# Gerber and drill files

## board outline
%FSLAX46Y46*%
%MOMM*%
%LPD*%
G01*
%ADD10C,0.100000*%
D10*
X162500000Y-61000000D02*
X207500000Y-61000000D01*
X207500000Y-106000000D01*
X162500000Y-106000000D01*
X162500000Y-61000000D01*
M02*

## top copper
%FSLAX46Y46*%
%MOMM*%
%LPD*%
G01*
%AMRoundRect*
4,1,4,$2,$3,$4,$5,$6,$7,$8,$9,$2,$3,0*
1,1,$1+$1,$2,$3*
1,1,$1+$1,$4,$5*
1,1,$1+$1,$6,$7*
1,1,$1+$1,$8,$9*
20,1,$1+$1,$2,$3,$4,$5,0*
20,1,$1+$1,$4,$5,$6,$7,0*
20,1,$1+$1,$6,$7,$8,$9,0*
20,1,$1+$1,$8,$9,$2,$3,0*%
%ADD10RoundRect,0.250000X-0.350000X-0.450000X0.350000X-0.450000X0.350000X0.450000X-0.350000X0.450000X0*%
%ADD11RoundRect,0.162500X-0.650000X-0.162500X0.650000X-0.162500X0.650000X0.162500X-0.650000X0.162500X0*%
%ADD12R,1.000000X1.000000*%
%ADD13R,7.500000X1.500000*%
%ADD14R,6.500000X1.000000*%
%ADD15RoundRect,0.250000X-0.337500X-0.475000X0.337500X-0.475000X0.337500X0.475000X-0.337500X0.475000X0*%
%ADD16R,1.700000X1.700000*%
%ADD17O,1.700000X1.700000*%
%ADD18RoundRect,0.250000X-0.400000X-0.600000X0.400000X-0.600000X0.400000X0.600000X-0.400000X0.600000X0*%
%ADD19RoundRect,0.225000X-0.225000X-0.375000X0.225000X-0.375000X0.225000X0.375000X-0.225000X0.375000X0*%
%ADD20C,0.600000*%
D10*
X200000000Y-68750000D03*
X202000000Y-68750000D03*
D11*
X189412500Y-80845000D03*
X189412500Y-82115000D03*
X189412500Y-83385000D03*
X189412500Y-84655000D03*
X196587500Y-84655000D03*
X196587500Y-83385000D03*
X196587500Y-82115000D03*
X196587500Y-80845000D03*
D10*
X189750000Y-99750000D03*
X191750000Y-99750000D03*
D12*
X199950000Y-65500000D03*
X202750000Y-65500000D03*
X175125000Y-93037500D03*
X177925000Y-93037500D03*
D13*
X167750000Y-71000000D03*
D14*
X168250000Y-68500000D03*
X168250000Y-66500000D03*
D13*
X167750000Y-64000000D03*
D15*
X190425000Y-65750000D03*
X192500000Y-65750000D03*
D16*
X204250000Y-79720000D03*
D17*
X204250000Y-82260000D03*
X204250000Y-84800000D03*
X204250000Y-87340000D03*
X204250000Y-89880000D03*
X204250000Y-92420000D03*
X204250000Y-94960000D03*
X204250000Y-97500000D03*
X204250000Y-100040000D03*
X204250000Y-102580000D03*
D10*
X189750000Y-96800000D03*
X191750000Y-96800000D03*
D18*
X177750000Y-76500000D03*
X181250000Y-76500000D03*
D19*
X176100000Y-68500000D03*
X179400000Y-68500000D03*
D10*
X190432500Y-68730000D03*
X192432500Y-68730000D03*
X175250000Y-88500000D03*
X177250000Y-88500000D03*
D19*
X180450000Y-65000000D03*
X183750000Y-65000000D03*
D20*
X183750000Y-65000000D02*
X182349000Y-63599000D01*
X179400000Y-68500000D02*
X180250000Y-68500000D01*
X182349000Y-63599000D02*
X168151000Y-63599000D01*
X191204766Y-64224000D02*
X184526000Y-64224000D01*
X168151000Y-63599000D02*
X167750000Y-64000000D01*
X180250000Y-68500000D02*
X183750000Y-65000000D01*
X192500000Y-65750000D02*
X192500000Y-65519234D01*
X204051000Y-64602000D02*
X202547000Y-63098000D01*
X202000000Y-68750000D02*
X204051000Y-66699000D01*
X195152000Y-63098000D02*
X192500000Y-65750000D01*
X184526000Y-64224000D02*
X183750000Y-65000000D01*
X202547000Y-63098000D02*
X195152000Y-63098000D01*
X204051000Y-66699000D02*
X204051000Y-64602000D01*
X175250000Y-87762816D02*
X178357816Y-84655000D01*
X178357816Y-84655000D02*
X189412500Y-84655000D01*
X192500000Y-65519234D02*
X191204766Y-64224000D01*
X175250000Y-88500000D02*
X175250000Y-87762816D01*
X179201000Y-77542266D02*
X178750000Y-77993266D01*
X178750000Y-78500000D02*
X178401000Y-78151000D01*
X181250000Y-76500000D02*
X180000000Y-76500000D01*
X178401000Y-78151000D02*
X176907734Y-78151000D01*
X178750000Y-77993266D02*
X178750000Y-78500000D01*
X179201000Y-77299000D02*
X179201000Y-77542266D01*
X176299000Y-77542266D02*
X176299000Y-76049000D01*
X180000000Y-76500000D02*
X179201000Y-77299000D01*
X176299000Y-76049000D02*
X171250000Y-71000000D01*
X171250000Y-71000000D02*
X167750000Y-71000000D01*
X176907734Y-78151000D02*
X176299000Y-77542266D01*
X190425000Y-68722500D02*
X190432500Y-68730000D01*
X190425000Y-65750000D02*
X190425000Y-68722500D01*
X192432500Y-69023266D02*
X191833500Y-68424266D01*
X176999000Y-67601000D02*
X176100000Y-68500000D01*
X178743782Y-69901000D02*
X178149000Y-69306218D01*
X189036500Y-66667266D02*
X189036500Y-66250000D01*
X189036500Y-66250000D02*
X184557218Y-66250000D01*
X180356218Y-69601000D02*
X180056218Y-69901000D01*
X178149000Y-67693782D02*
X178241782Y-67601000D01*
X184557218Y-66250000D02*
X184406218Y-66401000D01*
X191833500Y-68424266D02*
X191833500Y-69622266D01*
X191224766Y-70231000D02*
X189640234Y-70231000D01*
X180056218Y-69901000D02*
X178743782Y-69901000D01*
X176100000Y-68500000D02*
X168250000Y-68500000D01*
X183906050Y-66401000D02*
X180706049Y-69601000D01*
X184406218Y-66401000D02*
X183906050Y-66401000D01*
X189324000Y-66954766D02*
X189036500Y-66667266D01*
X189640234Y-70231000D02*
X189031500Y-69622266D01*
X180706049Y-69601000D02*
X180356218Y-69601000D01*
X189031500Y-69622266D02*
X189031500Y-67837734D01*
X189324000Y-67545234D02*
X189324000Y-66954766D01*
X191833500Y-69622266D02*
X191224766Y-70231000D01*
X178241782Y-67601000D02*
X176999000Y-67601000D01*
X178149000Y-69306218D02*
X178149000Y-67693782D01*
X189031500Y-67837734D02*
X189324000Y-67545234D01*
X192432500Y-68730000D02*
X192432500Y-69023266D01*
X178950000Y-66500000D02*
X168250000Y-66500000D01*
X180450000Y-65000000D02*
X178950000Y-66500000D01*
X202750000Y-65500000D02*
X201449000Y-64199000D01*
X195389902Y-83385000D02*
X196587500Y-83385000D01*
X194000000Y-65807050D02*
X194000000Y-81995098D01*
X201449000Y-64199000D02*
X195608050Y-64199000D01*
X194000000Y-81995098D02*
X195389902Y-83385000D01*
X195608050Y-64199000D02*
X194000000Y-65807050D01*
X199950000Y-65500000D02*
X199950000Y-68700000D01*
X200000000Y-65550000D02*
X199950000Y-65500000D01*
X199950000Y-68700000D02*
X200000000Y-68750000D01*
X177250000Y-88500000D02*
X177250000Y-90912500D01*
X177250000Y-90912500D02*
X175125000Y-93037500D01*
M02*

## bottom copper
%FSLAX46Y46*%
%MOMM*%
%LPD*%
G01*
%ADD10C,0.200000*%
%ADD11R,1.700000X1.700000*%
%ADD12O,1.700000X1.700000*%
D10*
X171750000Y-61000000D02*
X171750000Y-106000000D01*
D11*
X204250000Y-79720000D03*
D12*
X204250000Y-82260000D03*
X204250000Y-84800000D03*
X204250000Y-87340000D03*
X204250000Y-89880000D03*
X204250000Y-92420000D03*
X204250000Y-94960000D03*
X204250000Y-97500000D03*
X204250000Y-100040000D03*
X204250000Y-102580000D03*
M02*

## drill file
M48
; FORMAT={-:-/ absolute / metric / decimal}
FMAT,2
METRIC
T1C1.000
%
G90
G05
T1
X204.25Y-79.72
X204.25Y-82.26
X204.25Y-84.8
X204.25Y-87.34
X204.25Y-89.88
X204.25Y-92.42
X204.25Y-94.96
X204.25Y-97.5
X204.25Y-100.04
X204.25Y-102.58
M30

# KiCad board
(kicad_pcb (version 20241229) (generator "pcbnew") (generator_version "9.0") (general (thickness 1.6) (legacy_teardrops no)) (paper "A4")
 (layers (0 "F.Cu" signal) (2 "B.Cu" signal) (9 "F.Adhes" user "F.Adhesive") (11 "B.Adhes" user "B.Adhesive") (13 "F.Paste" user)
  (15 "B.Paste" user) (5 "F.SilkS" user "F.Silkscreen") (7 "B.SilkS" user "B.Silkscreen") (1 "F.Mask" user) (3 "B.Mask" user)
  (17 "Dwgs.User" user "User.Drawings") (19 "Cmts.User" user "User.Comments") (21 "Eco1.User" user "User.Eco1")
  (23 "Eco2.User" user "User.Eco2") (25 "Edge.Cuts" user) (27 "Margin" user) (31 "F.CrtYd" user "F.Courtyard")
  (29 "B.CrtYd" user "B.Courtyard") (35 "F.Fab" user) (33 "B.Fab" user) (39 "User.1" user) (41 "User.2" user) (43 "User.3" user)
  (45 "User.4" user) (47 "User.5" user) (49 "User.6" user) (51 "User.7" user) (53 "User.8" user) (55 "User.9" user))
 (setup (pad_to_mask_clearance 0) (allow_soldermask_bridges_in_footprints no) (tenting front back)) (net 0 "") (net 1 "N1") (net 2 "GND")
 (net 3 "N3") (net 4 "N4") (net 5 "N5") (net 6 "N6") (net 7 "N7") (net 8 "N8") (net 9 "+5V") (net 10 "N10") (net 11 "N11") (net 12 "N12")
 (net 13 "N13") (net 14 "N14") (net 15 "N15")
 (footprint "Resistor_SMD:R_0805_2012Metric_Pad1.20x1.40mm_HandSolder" (layer "F.Cu") (at 201 68.75)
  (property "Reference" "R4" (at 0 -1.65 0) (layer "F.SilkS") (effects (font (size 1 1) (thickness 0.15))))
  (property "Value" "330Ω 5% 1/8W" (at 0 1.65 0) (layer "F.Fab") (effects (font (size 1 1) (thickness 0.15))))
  (pad "1" smd roundrect (at -1 0) (size 1.2 1.4) (layers "F.Cu" "F.Mask" "F.Paste") (roundrect_rratio 0.208333) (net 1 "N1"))
  (pad "2" smd roundrect (at 1 0) (size 1.2 1.4) (layers "F.Cu" "F.Mask" "F.Paste") (roundrect_rratio 0.208333) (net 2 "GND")))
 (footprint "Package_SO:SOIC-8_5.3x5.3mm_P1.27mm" (layer "F.Cu") (at 193 82.75)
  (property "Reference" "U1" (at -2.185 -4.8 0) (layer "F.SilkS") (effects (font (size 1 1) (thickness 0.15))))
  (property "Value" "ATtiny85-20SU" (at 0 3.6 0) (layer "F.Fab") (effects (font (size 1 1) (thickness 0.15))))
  (pad "1" smd roundrect (at -3.5875 -1.905) (size 1.625 0.65) (layers "F.Cu" "F.Mask" "F.Paste") (roundrect_rratio 0.25) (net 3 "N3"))
  (pad "2" smd roundrect (at -3.5875 -0.635) (size 1.625 0.65) (layers "F.Cu" "F.Mask" "F.Paste") (roundrect_rratio 0.25) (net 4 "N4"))
  (pad "3" smd roundrect (at -3.5875 0.635) (size 1.625 0.65) (layers "F.Cu" "F.Mask" "F.Paste") (roundrect_rratio 0.25) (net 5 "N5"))
  (pad "4" smd roundrect (at -3.5875 1.905) (size 1.625 0.65) (layers "F.Cu" "F.Mask" "F.Paste") (roundrect_rratio 0.25) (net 2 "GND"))
  (pad "5" smd roundrect (at 3.5875 1.905) (size 1.625 0.65) (layers "F.Cu" "F.Mask" "F.Paste") (roundrect_rratio 0.25) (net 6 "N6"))
  (pad "6" smd roundrect (at 3.5875 0.635) (size 1.625 0.65) (layers "F.Cu" "F.Mask" "F.Paste") (roundrect_rratio 0.25) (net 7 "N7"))
  (pad "7" smd roundrect (at 3.5875 -0.635) (size 1.625 0.65) (layers "F.Cu" "F.Mask" "F.Paste") (roundrect_rratio 0.25) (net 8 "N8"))
  (pad "8" smd roundrect (at 3.5875 -1.905) (size 1.625 0.65) (layers "F.Cu" "F.Mask" "F.Paste") (roundrect_rratio 0.25) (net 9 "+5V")))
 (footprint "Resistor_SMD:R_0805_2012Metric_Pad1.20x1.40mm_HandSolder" (layer "F.Cu") (at 190.75 99.75)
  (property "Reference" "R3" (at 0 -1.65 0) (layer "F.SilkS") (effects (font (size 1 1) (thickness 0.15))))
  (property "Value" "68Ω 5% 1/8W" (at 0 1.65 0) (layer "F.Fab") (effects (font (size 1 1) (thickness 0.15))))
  (pad "1" smd roundrect (at -1 0) (size 1.2 1.4) (layers "F.Cu" "F.Mask" "F.Paste") (roundrect_rratio 0.208333) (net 5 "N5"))
  (pad "2" smd roundrect (at 1 0) (size 1.2 1.4) (layers "F.Cu" "F.Mask" "F.Paste") (roundrect_rratio 0.208333) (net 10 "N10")))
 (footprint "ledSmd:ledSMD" (layer "F.Cu") (at 201.75 65.5)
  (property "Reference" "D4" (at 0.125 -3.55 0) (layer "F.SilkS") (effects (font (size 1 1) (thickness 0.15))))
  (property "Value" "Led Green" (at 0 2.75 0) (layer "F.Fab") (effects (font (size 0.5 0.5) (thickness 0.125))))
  (pad "1" smd rect (at -1.8 0) (size 1 1) (layers "F.Cu" "F.Mask" "F.Paste") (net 1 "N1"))
  (pad "2" smd rect (at 1 0) (size 1 1) (layers "F.Cu" "F.Mask" "F.Paste") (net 7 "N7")))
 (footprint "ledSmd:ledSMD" (layer "F.Cu") (at 176.925 93.0375)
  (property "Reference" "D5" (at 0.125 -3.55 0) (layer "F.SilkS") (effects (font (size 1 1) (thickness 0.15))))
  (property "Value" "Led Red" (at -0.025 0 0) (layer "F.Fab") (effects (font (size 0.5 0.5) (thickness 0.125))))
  (pad "1" smd rect (at -1.8 0) (size 1 1) (layers "F.Cu" "F.Mask" "F.Paste") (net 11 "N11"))
  (pad "2" smd rect (at 1 0) (size 1 1) (layers "F.Cu" "F.Mask" "F.Paste") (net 9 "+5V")))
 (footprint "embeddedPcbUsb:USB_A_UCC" (layer "F.Cu") (at 167.95 67.5)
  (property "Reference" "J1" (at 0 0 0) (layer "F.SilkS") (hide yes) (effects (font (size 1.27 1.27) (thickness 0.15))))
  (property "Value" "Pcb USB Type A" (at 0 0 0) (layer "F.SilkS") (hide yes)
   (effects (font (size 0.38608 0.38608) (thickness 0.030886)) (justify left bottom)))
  (pad "1" smd rect (at -0.2 3.5) (size 7.5 1.5) (layers "F.Cu" "F.Mask" "F.Paste") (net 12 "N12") (solder_mask_margin 0.1016))
  (pad "2" smd rect (at 0.3 1) (size 6.5 1) (layers "F.Cu" "F.Mask" "F.Paste") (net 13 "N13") (solder_mask_margin 0.1016))
  (pad "3" smd rect (at 0.3 -1) (size 6.5 1) (layers "F.Cu" "F.Mask" "F.Paste") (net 10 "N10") (solder_mask_margin 0.1016))
  (pad "4" smd rect (at -0.2 -3.5) (size 7.5 1.5) (layers "F.Cu" "F.Mask" "F.Paste") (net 2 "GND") (solder_mask_margin 0.1016)))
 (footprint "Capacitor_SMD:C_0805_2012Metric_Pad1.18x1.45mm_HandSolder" (layer "F.Cu") (at 191.4625 65.75)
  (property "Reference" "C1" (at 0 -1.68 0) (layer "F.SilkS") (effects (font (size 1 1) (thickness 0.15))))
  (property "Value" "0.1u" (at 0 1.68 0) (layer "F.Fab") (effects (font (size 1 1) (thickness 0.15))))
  (pad "1" smd roundrect (at -1.0375 0) (size 1.175 1.45) (layers "F.Cu" "F.Mask" "F.Paste") (roundrect_rratio 0.212766) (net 9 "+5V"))
  (pad "2" smd roundrect (at 1.0375 0) (size 1.175 1.45) (layers "F.Cu" "F.Mask" "F.Paste") (roundrect_rratio 0.212766) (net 2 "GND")))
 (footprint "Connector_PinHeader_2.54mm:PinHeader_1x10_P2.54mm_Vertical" (layer "F.Cu") (at 204.25 79.72)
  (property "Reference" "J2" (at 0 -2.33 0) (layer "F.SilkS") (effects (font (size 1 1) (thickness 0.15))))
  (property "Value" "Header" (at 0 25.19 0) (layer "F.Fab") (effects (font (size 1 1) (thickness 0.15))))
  (pad "1" thru_hole rect (at 0 0) (size 1.7 1.7) (drill 1) (layers "*.Cu" "*.Mask") (remove_unused_layers no) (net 9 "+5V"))
  (pad "2" thru_hole oval (at 0 2.54) (size 1.7 1.7) (drill 1) (layers "*.Cu" "*.Mask") (remove_unused_layers no) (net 2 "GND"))
  (pad "3" thru_hole oval (at 0 5.08) (size 1.7 1.7) (drill 1) (layers "*.Cu" "*.Mask") (remove_unused_layers no) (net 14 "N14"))
  (pad "4" thru_hole oval (at 0 7.62) (size 1.7 1.7) (drill 1) (layers "*.Cu" "*.Mask") (remove_unused_layers no) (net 6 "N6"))
  (pad "5" thru_hole oval (at 0 10.16) (size 1.7 1.7) (drill 1) (layers "*.Cu" "*.Mask") (remove_unused_layers no) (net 7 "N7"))
  (pad "6" thru_hole oval (at 0 12.7) (size 1.7 1.7) (drill 1) (layers "*.Cu" "*.Mask") (remove_unused_layers no) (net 8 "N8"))
  (pad "7" thru_hole oval (at 0 15.24) (size 1.7 1.7) (drill 1) (layers "*.Cu" "*.Mask") (remove_unused_layers no) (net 4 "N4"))
  (pad "8" thru_hole oval (at 0 17.78) (size 1.7 1.7) (drill 1) (layers "*.Cu" "*.Mask") (remove_unused_layers no) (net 5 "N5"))
  (pad "9" thru_hole oval (at 0 20.32) (size 1.7 1.7) (drill 1) (layers "*.Cu" "*.Mask") (remove_unused_layers no) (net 3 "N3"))
  (pad "10" thru_hole oval (at 0 22.86) (size 1.7 1.7) (drill 1) (layers "*.Cu" "*.Mask") (remove_unused_layers no) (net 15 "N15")))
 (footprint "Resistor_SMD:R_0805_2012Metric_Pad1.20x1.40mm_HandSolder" (layer "F.Cu") (at 190.75 96.8)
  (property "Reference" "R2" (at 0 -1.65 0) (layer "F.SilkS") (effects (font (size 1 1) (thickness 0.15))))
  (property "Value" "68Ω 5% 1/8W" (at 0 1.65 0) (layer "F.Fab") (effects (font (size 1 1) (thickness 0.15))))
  (pad "1" smd roundrect (at -1 0) (size 1.2 1.4) (layers "F.Cu" "F.Mask" "F.Paste") (roundrect_rratio 0.208333) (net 4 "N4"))
  (pad "2" smd roundrect (at 1 0) (size 1.2 1.4) (layers "F.Cu" "F.Mask" "F.Paste") (roundrect_rratio 0.208333) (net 13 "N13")))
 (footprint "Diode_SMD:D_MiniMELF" (layer "F.Cu") (at 179.5 76.5)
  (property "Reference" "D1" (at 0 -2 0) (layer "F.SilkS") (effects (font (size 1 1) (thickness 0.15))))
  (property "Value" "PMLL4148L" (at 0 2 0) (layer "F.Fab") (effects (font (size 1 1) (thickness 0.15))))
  (pad "1" smd roundrect (at -1.75 0) (size 1.3 1.7) (layers "F.Cu" "F.Mask" "F.Paste") (roundrect_rratio 0.1923076923) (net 9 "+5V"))
  (pad "2" smd roundrect (at 1.75 0) (size 1.3 1.7) (layers "F.Cu" "F.Mask" "F.Paste") (roundrect_rratio 0.1923076923) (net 12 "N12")))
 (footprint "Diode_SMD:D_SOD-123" (layer "F.Cu") (at 177.75 68.5)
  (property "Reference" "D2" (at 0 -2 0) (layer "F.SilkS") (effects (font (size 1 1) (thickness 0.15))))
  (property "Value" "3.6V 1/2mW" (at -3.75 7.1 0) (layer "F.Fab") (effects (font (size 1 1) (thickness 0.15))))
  (pad "1" smd roundrect (at -1.65 0) (size 0.9 1.2) (layers "F.Cu" "F.Mask" "F.Paste") (roundrect_rratio 0.25) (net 13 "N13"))
  (pad "2" smd roundrect (at 1.65 0) (size 0.9 1.2) (layers "F.Cu" "F.Mask" "F.Paste") (roundrect_rratio 0.25) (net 2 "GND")))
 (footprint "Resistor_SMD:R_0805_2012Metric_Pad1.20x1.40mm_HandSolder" (layer "F.Cu") (at 191.4325 68.73)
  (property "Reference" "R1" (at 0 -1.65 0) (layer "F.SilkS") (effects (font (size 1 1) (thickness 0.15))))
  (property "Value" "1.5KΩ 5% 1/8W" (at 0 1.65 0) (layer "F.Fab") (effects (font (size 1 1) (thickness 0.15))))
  (pad "1" smd roundrect (at -1 0) (size 1.2 1.4) (layers "F.Cu" "F.Mask" "F.Paste") (roundrect_rratio 0.208333) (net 9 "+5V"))
  (pad "2" smd roundrect (at 1 0) (size 1.2 1.4) (layers "F.Cu" "F.Mask" "F.Paste") (roundrect_rratio 0.208333) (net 13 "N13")))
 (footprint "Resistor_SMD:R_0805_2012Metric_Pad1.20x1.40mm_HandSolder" (layer "F.Cu") (at 176.25 88.5)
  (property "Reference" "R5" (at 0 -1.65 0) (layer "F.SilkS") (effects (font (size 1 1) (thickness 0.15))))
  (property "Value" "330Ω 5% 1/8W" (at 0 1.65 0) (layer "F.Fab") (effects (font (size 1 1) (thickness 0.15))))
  (pad "1" smd roundrect (at -1 0) (size 1.2 1.4) (layers "F.Cu" "F.Mask" "F.Paste") (roundrect_rratio 0.208333) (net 2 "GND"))
  (pad "2" smd roundrect (at 1 0) (size 1.2 1.4) (layers "F.Cu" "F.Mask" "F.Paste") (roundrect_rratio 0.208333) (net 11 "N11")))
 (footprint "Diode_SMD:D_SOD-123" (layer "F.Cu") (at 182.1 65)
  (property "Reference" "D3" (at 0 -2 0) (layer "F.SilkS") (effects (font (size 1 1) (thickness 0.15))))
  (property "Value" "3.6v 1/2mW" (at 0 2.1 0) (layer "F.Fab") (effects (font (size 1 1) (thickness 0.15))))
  (pad "1" smd roundrect (at -1.65 0) (size 0.9 1.2) (layers "F.Cu" "F.Mask" "F.Paste") (roundrect_rratio 0.25) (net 10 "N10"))
  (pad "2" smd roundrect (at 1.65 0) (size 0.9 1.2) (layers "F.Cu" "F.Mask" "F.Paste") (roundrect_rratio 0.25) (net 2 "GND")))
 (gr_line (start 171.75 61) (end 171.75 106) (stroke (width 0.2) (type default)) (layer "B.Cu"))
 (gr_rect (start 162.5 61) (end 207.5 106) (stroke (width 0.1) (type default)) (fill no) (layer "Edge.Cuts"))
 (segment (start 183.75 65) (end 182.349 63.599) (width 0.6) (layer "F.Cu") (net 2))
 (segment (start 179.4 68.5) (end 180.25 68.5) (width 0.6) (layer "F.Cu") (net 2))
 (segment (start 182.349 63.599) (end 168.151 63.599) (width 0.6) (layer "F.Cu") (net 2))
 (segment (start 191.204766 64.224) (end 184.526 64.224) (width 0.6) (layer "F.Cu") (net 2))
 (segment (start 168.151 63.599) (end 167.75 64) (width 0.6) (layer "F.Cu") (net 2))
 (segment (start 180.25 68.5) (end 183.75 65) (width 0.6) (layer "F.Cu") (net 2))
 (segment (start 192.5 65.75) (end 192.5 65.519234) (width 0.6) (layer "F.Cu") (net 2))
 (segment (start 204.051 64.602) (end 202.547 63.098) (width 0.6) (layer "F.Cu") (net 2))
 (segment (start 202 68.75) (end 204.051 66.699) (width 0.6) (layer "F.Cu") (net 2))
 (segment (start 195.152 63.098) (end 192.5 65.75) (width 0.6) (layer "F.Cu") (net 2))
 (segment (start 184.526 64.224) (end 183.75 65) (width 0.6) (layer "F.Cu") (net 2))
 (segment (start 202.547 63.098) (end 195.152 63.098) (width 0.6) (layer "F.Cu") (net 2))
 (segment (start 204.051 66.699) (end 204.051 64.602) (width 0.6) (layer "F.Cu") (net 2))
 (segment (start 175.25 87.762816) (end 178.357816 84.655) (width 0.6) (layer "F.Cu") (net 2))
 (segment (start 178.357816 84.655) (end 189.4125 84.655) (width 0.6) (layer "F.Cu") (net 2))
 (segment (start 192.5 65.519234) (end 191.204766 64.224) (width 0.6) (layer "F.Cu") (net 2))
 (segment (start 175.25 88.5) (end 175.25 87.762816) (width 0.6) (layer "F.Cu") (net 2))
 (segment (start 179.201 77.542266) (end 178.75 77.993266) (width 0.6) (layer "F.Cu") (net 12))
 (segment (start 178.75 78.5) (end 178.401 78.151) (width 0.6) (layer "F.Cu") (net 12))
 (segment (start 181.25 76.5) (end 180 76.5) (width 0.6) (layer "F.Cu") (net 12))
 (segment (start 178.401 78.151) (end 176.907734 78.151) (width 0.6) (layer "F.Cu") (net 12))
 (segment (start 178.75 77.993266) (end 178.75 78.5) (width 0.6) (layer "F.Cu") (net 12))
 (segment (start 179.201 77.299) (end 179.201 77.542266) (width 0.6) (layer "F.Cu") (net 12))
 (segment (start 176.299 77.542266) (end 176.299 76.049) (width 0.6) (layer "F.Cu") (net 12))
 (segment (start 180 76.5) (end 179.201 77.299) (width 0.6) (layer "F.Cu") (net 12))
 (segment (start 176.299 76.049) (end 171.25 71) (width 0.6) (layer "F.Cu") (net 12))
 (segment (start 171.25 71) (end 167.75 71) (width 0.6) (layer "F.Cu") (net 12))
 (segment (start 176.907734 78.151) (end 176.299 77.542266) (width 0.6) (layer "F.Cu") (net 12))
 (segment (start 190.425 68.7225) (end 190.4325 68.73) (width 0.6) (layer "F.Cu") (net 9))
 (segment (start 190.425 65.75) (end 190.425 68.7225) (width 0.6) (layer "F.Cu") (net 9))
 (segment (start 192.4325 69.023266) (end 191.8335 68.424266) (width 0.6) (layer "F.Cu") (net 13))
 (segment (start 176.999 67.601) (end 176.1 68.5) (width 0.6) (layer "F.Cu") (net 13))
 (segment (start 178.743782 69.901) (end 178.149 69.306218) (width 0.6) (layer "F.Cu") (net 13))
 (segment (start 189.0365 66.667266) (end 189.0365 66.25) (width 0.6) (layer "F.Cu") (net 13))
 (segment (start 189.0365 66.25) (end 184.557218 66.25) (width 0.6) (layer "F.Cu") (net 13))
 (segment (start 180.356218 69.601) (end 180.056218 69.901) (width 0.6) (layer "F.Cu") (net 13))
 (segment (start 178.149 67.693782) (end 178.241782 67.601) (width 0.6) (layer "F.Cu") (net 13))
 (segment (start 184.557218 66.25) (end 184.406218 66.401) (width 0.6) (layer "F.Cu") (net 13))
 (segment (start 191.8335 68.424266) (end 191.8335 69.622266) (width 0.6) (layer "F.Cu") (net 13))
 (segment (start 191.224766 70.231) (end 189.640234 70.231) (width 0.6) (layer "F.Cu") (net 13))
 (segment (start 180.056218 69.901) (end 178.743782 69.901) (width 0.6) (layer "F.Cu") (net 13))
 (segment (start 176.1 68.5) (end 168.25 68.5) (width 0.6) (layer "F.Cu") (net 13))
 (segment (start 183.90605 66.401) (end 180.706049 69.601) (width 0.6) (layer "F.Cu") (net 13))
 (segment (start 184.406218 66.401) (end 183.90605 66.401) (width 0.6) (layer "F.Cu") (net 13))
 (segment (start 189.324 66.954766) (end 189.0365 66.667266) (width 0.6) (layer "F.Cu") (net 13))
 (segment (start 189.640234 70.231) (end 189.0315 69.622266) (width 0.6) (layer "F.Cu") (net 13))
 (segment (start 180.706049 69.601) (end 180.356218 69.601) (width 0.6) (layer "F.Cu") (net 13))
 (segment (start 189.0315 69.622266) (end 189.0315 67.837734) (width 0.6) (layer "F.Cu") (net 13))
 (segment (start 189.324 67.545234) (end 189.324 66.954766) (width 0.6) (layer "F.Cu") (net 13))
 (segment (start 191.8335 69.622266) (end 191.224766 70.231) (width 0.6) (layer "F.Cu") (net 13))
 (segment (start 178.241782 67.601) (end 176.999 67.601) (width 0.6) (layer "F.Cu") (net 13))
 (segment (start 178.149 69.306218) (end 178.149 67.693782) (width 0.6) (layer "F.Cu") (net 13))
 (segment (start 189.0315 67.837734) (end 189.324 67.545234) (width 0.6) (layer "F.Cu") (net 13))
 (segment (start 192.4325 68.73) (end 192.4325 69.023266) (width 0.6) (layer "F.Cu") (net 13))
 (segment (start 178.95 66.5) (end 168.25 66.5) (width 0.6) (layer "F.Cu") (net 10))
 (segment (start 180.45 65) (end 178.95 66.5) (width 0.6) (layer "F.Cu") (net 10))
 (segment (start 202.75 65.5) (end 201.449 64.199) (width 0.6) (layer "F.Cu") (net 7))
 (segment (start 195.389902 83.385) (end 196.5875 83.385) (width 0.6) (layer "F.Cu") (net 7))
 (segment (start 194 65.80705) (end 194 81.995098) (width 0.6) (layer "F.Cu") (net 7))
 (segment (start 201.449 64.199) (end 195.60805 64.199) (width 0.6) (layer "F.Cu") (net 7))
 (segment (start 194 81.995098) (end 195.389902 83.385) (width 0.6) (layer "F.Cu") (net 7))
 (segment (start 195.60805 64.199) (end 194 65.80705) (width 0.6) (layer "F.Cu") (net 7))
 (segment (start 199.95 65.5) (end 199.95 68.7) (width 0.6) (layer "F.Cu") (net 1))
 (segment (start 200 65.55) (end 199.95 65.5) (width 0.6) (layer "F.Cu") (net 1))
 (segment (start 199.95 68.7) (end 200 68.75) (width 0.6) (layer "F.Cu") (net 1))
 (segment (start 177.25 88.5) (end 177.25 90.9125) (width 0.6) (layer "F.Cu") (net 11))
 (segment (start 177.25 90.9125) (end 175.125 93.0375) (width 0.6) (layer "F.Cu") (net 11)))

